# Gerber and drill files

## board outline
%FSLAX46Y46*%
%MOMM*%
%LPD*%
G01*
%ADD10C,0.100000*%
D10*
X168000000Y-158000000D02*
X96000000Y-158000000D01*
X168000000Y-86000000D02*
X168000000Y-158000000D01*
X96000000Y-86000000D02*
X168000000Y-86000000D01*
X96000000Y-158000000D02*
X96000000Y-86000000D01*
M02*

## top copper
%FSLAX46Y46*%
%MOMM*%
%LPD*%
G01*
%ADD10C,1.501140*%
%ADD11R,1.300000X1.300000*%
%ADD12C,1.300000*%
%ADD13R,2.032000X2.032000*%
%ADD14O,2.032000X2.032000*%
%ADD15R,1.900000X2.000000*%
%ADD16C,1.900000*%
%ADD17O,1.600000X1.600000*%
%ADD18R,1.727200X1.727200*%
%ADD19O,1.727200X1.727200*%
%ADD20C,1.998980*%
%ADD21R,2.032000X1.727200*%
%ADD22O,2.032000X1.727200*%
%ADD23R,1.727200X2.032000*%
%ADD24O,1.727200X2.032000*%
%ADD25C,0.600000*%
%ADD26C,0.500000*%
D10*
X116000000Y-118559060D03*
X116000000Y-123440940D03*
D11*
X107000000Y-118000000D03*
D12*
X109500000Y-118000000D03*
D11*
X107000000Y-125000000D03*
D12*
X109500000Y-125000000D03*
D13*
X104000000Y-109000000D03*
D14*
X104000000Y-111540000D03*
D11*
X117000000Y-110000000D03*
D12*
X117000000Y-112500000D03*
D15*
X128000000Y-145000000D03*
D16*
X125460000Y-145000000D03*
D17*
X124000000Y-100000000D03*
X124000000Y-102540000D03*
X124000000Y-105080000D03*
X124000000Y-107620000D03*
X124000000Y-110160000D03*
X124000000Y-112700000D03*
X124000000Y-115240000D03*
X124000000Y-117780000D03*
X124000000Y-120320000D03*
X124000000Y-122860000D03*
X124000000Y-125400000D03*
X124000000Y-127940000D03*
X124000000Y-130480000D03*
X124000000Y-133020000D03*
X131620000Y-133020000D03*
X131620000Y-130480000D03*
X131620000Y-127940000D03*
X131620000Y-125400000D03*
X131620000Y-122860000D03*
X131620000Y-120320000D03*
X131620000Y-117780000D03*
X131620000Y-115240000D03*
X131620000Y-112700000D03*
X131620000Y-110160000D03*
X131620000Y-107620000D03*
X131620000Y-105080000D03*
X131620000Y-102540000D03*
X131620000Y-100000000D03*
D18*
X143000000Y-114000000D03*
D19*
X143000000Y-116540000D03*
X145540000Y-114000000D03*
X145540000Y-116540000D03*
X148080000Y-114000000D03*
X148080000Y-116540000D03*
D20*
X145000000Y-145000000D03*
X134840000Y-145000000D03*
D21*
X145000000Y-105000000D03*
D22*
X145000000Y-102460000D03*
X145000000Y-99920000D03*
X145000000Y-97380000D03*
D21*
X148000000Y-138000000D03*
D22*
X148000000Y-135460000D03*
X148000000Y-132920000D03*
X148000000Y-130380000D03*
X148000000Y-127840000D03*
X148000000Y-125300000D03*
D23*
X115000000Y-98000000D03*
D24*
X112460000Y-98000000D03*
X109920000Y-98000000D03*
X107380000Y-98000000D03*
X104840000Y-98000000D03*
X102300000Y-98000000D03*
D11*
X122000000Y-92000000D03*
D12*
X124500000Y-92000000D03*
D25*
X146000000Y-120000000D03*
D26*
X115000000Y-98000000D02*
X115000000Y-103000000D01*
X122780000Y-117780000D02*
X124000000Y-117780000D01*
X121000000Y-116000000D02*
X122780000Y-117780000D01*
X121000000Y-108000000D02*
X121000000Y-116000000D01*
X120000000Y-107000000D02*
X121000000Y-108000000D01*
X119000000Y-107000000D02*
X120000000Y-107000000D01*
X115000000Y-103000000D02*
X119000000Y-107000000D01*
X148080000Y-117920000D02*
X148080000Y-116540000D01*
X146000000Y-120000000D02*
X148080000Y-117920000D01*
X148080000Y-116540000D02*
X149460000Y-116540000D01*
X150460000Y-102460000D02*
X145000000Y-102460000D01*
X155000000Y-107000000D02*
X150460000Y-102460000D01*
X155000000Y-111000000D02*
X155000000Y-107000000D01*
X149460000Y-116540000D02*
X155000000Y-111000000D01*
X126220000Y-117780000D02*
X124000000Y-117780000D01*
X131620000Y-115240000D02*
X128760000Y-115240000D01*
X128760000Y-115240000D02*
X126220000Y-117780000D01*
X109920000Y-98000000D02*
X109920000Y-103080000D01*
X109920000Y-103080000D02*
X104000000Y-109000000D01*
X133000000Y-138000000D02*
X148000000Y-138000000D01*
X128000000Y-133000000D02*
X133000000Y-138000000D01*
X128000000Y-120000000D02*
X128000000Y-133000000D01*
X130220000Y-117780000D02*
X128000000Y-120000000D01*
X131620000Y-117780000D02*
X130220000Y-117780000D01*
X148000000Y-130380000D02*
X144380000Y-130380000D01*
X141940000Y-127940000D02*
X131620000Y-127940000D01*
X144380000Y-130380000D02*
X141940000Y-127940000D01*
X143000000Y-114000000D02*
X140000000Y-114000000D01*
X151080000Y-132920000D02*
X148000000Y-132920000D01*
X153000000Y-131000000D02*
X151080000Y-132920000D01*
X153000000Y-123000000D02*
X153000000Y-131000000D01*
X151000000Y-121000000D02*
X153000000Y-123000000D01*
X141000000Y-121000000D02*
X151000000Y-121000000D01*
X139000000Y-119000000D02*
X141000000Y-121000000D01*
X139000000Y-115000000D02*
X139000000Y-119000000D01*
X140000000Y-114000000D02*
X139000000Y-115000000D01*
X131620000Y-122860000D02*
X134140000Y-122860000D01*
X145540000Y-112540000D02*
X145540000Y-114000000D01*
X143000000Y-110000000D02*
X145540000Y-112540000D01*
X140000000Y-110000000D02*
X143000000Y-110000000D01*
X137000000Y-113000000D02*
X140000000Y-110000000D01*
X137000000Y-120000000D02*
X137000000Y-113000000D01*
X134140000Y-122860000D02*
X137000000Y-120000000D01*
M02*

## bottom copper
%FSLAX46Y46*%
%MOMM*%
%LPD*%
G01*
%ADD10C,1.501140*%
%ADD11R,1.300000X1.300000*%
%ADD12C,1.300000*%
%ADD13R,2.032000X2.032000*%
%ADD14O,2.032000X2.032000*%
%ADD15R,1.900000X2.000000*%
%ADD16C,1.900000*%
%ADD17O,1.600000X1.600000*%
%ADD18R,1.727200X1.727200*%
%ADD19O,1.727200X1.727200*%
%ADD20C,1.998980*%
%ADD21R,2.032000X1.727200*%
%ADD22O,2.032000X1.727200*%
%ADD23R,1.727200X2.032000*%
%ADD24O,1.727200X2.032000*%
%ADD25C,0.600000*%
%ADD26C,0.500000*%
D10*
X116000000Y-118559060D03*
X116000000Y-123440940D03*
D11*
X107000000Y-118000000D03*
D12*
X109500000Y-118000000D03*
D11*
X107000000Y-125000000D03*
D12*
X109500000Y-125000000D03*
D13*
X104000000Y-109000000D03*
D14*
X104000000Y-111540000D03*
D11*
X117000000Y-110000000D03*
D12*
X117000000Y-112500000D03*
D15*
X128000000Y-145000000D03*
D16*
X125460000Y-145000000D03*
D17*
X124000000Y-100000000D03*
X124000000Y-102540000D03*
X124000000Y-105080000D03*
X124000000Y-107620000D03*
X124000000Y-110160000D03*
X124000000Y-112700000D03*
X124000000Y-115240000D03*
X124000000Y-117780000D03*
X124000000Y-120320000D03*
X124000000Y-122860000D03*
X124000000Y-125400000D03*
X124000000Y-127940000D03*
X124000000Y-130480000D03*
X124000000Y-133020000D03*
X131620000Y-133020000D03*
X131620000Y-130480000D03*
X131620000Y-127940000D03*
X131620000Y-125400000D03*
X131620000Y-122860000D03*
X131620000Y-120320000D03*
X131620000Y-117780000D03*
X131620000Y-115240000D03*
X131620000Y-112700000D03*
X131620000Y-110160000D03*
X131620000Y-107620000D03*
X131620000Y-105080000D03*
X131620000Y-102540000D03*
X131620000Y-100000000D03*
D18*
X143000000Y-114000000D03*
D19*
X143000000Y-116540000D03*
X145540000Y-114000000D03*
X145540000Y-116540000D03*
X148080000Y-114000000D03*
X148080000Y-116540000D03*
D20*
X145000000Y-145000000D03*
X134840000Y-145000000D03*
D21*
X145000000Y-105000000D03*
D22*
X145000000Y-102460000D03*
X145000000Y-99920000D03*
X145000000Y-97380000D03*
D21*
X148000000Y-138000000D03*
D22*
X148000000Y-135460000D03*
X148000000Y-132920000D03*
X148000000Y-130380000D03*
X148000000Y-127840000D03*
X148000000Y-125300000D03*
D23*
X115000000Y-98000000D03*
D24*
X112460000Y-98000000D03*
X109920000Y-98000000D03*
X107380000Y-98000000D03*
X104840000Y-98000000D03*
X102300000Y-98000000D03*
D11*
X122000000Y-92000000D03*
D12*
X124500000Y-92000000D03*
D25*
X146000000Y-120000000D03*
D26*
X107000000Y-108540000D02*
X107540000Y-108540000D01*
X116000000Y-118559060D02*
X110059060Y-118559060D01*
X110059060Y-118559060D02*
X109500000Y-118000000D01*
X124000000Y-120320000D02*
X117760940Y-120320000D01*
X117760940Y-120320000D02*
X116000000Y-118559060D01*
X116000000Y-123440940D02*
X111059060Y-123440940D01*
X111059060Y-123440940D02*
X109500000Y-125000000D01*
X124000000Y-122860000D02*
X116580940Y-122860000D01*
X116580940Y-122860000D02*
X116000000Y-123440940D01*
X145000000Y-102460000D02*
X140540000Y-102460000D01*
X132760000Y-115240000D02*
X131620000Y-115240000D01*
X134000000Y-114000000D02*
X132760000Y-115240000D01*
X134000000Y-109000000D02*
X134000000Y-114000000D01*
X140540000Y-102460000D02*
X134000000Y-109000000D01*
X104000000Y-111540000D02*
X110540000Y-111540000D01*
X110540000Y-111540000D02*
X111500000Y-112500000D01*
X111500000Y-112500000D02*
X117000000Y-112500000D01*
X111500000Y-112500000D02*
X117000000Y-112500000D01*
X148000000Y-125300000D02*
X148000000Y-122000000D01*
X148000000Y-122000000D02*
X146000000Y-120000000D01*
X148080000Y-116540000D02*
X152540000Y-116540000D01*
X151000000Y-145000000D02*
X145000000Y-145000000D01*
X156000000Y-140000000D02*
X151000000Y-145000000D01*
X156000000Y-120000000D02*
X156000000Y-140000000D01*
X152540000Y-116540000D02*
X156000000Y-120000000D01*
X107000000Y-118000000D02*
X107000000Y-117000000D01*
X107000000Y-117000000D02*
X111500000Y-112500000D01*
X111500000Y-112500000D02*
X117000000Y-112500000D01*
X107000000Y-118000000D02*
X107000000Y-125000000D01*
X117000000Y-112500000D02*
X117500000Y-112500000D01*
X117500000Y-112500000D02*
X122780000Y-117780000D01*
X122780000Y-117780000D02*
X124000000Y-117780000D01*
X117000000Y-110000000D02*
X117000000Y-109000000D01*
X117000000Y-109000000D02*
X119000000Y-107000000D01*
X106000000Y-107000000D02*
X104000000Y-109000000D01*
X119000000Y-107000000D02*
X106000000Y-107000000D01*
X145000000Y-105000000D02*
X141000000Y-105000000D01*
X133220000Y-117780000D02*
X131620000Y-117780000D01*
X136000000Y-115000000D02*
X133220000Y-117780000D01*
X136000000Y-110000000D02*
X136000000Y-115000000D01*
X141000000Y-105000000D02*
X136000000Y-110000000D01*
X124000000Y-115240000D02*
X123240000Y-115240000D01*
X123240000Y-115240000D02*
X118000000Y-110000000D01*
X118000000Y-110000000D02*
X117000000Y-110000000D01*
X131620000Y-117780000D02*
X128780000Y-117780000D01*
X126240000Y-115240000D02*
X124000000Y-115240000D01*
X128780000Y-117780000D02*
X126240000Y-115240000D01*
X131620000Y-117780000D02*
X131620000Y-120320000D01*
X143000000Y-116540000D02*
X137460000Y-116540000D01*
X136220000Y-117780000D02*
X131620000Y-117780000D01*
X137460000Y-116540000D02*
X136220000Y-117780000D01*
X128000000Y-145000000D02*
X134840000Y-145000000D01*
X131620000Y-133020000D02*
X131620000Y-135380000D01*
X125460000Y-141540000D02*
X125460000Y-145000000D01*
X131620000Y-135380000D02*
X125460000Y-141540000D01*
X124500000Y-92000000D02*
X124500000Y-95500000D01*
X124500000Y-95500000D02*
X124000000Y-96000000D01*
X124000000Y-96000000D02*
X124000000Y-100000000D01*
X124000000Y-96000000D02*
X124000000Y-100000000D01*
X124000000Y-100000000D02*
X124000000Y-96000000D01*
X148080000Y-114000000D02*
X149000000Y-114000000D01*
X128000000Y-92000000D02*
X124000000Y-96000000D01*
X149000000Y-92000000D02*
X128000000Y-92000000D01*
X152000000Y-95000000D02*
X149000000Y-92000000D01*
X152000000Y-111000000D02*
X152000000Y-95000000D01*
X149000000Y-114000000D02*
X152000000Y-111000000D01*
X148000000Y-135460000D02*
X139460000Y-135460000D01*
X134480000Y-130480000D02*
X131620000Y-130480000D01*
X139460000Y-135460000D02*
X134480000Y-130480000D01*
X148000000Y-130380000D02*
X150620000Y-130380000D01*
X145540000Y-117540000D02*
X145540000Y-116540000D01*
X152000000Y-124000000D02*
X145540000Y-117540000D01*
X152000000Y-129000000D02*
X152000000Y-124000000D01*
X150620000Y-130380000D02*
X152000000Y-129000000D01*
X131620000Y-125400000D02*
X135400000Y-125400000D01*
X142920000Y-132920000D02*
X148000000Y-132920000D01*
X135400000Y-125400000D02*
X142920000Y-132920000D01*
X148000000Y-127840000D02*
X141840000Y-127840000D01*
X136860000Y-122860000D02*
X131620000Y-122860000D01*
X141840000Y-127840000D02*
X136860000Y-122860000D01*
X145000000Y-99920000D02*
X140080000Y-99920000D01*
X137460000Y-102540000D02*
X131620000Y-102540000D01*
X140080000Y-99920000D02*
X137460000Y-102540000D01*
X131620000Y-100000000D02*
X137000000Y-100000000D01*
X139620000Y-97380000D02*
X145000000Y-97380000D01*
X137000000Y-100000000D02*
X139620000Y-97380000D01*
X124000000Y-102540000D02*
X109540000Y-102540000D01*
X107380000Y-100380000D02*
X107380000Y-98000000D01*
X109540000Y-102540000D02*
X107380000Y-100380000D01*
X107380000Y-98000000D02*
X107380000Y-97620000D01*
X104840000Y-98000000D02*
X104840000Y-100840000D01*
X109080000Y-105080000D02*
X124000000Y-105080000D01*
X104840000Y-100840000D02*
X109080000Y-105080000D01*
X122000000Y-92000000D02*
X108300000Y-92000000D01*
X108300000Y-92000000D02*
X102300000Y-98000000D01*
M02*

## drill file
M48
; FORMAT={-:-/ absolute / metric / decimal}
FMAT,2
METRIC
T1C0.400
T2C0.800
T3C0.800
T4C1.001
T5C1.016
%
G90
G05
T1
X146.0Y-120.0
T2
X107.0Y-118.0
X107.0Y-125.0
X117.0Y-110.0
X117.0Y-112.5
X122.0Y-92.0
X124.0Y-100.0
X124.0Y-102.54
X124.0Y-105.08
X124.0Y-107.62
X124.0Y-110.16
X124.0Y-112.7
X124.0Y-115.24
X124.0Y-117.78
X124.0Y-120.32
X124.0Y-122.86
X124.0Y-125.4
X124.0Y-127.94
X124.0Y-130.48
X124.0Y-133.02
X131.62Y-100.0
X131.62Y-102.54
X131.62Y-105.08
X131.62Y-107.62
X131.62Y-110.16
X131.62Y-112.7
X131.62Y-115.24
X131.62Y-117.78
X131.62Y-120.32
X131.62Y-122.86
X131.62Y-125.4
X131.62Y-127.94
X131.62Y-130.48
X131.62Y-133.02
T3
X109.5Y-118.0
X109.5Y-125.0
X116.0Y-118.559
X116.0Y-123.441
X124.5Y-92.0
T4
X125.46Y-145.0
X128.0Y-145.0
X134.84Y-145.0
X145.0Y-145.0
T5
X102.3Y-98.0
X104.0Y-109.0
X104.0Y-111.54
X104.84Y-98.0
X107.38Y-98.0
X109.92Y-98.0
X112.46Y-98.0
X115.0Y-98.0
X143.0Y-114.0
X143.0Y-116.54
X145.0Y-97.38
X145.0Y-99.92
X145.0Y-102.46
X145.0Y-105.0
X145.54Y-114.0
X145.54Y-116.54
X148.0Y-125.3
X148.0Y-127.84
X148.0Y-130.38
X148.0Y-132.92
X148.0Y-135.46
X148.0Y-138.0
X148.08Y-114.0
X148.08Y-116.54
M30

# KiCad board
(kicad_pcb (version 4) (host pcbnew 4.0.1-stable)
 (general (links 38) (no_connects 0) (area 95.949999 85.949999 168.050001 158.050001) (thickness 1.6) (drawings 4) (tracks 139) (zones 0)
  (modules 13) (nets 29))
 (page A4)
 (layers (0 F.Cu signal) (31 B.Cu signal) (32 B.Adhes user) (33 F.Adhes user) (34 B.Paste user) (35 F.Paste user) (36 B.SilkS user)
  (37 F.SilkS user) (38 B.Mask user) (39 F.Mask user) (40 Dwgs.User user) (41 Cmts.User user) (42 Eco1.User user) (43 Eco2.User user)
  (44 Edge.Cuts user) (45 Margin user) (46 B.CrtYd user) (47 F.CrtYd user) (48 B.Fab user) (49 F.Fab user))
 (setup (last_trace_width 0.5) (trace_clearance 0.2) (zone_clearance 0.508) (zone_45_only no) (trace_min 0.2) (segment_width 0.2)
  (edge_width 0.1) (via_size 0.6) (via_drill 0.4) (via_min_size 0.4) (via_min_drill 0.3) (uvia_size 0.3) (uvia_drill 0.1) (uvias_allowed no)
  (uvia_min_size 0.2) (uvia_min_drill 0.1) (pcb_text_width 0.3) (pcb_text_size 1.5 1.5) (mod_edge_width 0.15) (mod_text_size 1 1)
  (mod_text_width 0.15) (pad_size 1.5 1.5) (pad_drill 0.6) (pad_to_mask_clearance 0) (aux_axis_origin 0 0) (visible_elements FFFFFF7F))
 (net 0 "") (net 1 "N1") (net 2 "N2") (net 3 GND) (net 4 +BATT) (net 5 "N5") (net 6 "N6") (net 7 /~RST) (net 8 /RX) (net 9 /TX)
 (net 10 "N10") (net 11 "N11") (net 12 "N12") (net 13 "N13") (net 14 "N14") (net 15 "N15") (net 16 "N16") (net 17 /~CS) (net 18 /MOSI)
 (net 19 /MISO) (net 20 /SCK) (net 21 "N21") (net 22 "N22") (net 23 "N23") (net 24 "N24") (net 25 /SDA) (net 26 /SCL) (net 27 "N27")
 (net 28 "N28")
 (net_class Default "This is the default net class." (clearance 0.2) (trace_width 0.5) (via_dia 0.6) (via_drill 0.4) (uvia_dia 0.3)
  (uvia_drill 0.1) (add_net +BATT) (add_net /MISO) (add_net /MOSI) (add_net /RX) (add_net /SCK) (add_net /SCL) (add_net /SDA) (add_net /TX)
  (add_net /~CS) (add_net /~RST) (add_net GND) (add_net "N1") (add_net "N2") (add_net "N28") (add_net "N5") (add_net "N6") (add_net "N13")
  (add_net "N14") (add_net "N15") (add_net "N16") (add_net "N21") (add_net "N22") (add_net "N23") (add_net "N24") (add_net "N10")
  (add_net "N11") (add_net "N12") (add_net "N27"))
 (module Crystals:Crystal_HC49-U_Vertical (layer F.Cu) (at 116 121 270)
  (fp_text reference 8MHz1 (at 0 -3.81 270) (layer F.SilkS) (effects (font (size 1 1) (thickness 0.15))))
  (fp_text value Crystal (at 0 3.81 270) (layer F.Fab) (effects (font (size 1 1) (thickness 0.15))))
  (pad 1 thru_hole circle (at -2.44094 0 270) (size 1.50114 1.50114) (drill 0.8001) (layers *.Cu *.Mask F.SilkS) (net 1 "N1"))
  (pad 2 thru_hole circle (at 2.44094 0 270) (size 1.50114 1.50114) (drill 0.8001) (layers *.Cu *.Mask F.SilkS) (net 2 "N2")))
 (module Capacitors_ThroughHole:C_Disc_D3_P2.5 (layer F.Cu) (at 107 118)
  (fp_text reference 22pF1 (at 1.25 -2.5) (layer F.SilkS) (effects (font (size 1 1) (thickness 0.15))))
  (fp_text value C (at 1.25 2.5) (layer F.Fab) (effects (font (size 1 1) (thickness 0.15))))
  (pad 1 thru_hole rect (at 0 0) (size 1.3 1.3) (drill 0.8) (layers *.Cu *.Mask F.SilkS) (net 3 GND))
  (pad 2 thru_hole circle (at 2.5 0) (size 1.3 1.3) (drill 0.8001) (layers *.Cu *.Mask F.SilkS) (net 1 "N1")))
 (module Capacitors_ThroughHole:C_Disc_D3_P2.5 (layer F.Cu) (at 107 125)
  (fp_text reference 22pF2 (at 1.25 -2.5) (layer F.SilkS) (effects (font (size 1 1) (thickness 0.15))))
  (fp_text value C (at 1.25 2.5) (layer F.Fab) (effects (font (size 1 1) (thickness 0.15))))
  (pad 1 thru_hole rect (at 0 0) (size 1.3 1.3) (drill 0.8) (layers *.Cu *.Mask F.SilkS) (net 3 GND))
  (pad 2 thru_hole circle (at 2.5 0) (size 1.3 1.3) (drill 0.8001) (layers *.Cu *.Mask F.SilkS) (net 2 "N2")))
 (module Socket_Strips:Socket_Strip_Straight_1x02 (layer F.Cu) (at 104 109 270)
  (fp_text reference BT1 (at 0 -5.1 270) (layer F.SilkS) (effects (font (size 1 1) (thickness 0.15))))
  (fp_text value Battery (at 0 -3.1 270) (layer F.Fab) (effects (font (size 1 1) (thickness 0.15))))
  (pad 1 thru_hole rect (at 0 0 270) (size 2.032 2.032) (drill 1.016) (layers *.Cu *.Mask F.SilkS) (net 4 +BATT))
  (pad 2 thru_hole oval (at 2.54 0 270) (size 2.032 2.032) (drill 1.016) (layers *.Cu *.Mask F.SilkS) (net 3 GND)))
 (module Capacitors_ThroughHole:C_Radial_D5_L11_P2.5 (layer F.Cu) (at 117 110 270)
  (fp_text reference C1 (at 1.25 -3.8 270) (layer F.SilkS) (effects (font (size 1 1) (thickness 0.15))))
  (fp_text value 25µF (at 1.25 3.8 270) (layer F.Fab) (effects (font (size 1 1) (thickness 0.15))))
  (pad 1 thru_hole rect (at 0 0 270) (size 1.3 1.3) (drill 0.8) (layers *.Cu *.Mask F.SilkS) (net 4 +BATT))
  (pad 2 thru_hole circle (at 2.5 0 270) (size 1.3 1.3) (drill 0.8) (layers *.Cu *.Mask F.SilkS) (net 3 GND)))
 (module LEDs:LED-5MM (layer F.Cu) (at 128 145 180)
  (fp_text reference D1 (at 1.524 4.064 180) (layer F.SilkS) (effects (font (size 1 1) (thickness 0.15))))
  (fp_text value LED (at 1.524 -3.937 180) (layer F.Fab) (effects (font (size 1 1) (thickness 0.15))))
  (pad 1 thru_hole rect (at 0 0 270) (size 2 1.9) (drill 1.00076) (layers *.Cu *.Mask F.SilkS) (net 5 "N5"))
  (pad 2 thru_hole circle (at 2.54 0 180) (size 1.9 1.9) (drill 1.00076) (layers *.Cu *.Mask F.SilkS) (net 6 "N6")))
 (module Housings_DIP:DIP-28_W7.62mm (layer F.Cu) (at 124 100)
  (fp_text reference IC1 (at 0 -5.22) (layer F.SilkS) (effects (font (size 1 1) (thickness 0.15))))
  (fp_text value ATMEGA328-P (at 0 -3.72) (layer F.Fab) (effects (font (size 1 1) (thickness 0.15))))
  (pad 1 thru_hole oval (at 0 0) (size 1.6 1.6) (drill 0.8) (layers *.Cu *.Mask F.SilkS) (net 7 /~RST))
  (pad 2 thru_hole oval (at 0 2.54) (size 1.6 1.6) (drill 0.8) (layers *.Cu *.Mask F.SilkS) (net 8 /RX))
  (pad 3 thru_hole oval (at 0 5.08) (size 1.6 1.6) (drill 0.8) (layers *.Cu *.Mask F.SilkS) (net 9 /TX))
  (pad 4 thru_hole oval (at 0 7.62) (size 1.6 1.6) (drill 0.8) (layers *.Cu *.Mask F.SilkS) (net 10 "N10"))
  (pad 5 thru_hole oval (at 0 10.16) (size 1.6 1.6) (drill 0.8) (layers *.Cu *.Mask F.SilkS) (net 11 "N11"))
  (pad 6 thru_hole oval (at 0 12.7) (size 1.6 1.6) (drill 0.8) (layers *.Cu *.Mask F.SilkS) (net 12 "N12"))
  (pad 7 thru_hole oval (at 0 15.24) (size 1.6 1.6) (drill 0.8) (layers *.Cu *.Mask F.SilkS) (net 4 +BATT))
  (pad 8 thru_hole oval (at 0 17.78) (size 1.6 1.6) (drill 0.8) (layers *.Cu *.Mask F.SilkS) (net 3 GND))
  (pad 9 thru_hole oval (at 0 20.32) (size 1.6 1.6) (drill 0.8) (layers *.Cu *.Mask F.SilkS) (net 1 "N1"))
  (pad 10 thru_hole oval (at 0 22.86) (size 1.6 1.6) (drill 0.8) (layers *.Cu *.Mask F.SilkS) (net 2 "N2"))
  (pad 11 thru_hole oval (at 0 25.4) (size 1.6 1.6) (drill 0.8) (layers *.Cu *.Mask F.SilkS) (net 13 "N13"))
  (pad 12 thru_hole oval (at 0 27.94) (size 1.6 1.6) (drill 0.8) (layers *.Cu *.Mask F.SilkS) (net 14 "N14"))
  (pad 13 thru_hole oval (at 0 30.48) (size 1.6 1.6) (drill 0.8) (layers *.Cu *.Mask F.SilkS) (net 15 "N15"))
  (pad 14 thru_hole oval (at 0 33.02) (size 1.6 1.6) (drill 0.8) (layers *.Cu *.Mask F.SilkS) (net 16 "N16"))
  (pad 15 thru_hole oval (at 7.62 33.02) (size 1.6 1.6) (drill 0.8) (layers *.Cu *.Mask F.SilkS) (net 6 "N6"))
  (pad 16 thru_hole oval (at 7.62 30.48) (size 1.6 1.6) (drill 0.8) (layers *.Cu *.Mask F.SilkS) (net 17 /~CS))
  (pad 17 thru_hole oval (at 7.62 27.94) (size 1.6 1.6) (drill 0.8) (layers *.Cu *.Mask F.SilkS) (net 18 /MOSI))
  (pad 18 thru_hole oval (at 7.62 25.4) (size 1.6 1.6) (drill 0.8) (layers *.Cu *.Mask F.SilkS) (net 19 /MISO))
  (pad 19 thru_hole oval (at 7.62 22.86) (size 1.6 1.6) (drill 0.8) (layers *.Cu *.Mask F.SilkS) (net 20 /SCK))
  (pad 20 thru_hole oval (at 7.62 20.32) (size 1.6 1.6) (drill 0.8) (layers *.Cu *.Mask F.SilkS) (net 4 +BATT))
  (pad 21 thru_hole oval (at 7.62 17.78) (size 1.6 1.6) (drill 0.8) (layers *.Cu *.Mask F.SilkS) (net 4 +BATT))
  (pad 22 thru_hole oval (at 7.62 15.24) (size 1.6 1.6) (drill 0.8) (layers *.Cu *.Mask F.SilkS) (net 3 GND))
  (pad 23 thru_hole oval (at 7.62 12.7) (size 1.6 1.6) (drill 0.8) (layers *.Cu *.Mask F.SilkS) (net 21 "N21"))
  (pad 24 thru_hole oval (at 7.62 10.16) (size 1.6 1.6) (drill 0.8) (layers *.Cu *.Mask F.SilkS) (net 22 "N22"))
  (pad 25 thru_hole oval (at 7.62 7.62) (size 1.6 1.6) (drill 0.8) (layers *.Cu *.Mask F.SilkS) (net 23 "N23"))
  (pad 26 thru_hole oval (at 7.62 5.08) (size 1.6 1.6) (drill 0.8) (layers *.Cu *.Mask F.SilkS) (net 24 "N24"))
  (pad 27 thru_hole oval (at 7.62 2.54) (size 1.6 1.6) (drill 0.8) (layers *.Cu *.Mask F.SilkS) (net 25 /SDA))
  (pad 28 thru_hole oval (at 7.62 0) (size 1.6 1.6) (drill 0.8) (layers *.Cu *.Mask F.SilkS) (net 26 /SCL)))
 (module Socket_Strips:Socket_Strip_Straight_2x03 (layer F.Cu) (at 143 114)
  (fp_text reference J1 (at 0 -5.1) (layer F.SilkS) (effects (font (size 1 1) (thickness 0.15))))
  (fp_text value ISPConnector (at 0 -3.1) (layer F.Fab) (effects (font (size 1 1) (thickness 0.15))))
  (pad 1 thru_hole rect (at 0 0) (size 1.7272 1.7272) (drill 1.016) (layers *.Cu *.Mask F.SilkS) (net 19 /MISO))
  (pad 2 thru_hole oval (at 0 2.54) (size 1.7272 1.7272) (drill 1.016) (layers *.Cu *.Mask F.SilkS) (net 4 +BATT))
  (pad 3 thru_hole oval (at 2.54 0) (size 1.7272 1.7272) (drill 1.016) (layers *.Cu *.Mask F.SilkS) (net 20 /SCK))
  (pad 4 thru_hole oval (at 2.54 2.54) (size 1.7272 1.7272) (drill 1.016) (layers *.Cu *.Mask F.SilkS) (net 18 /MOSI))
  (pad 5 thru_hole oval (at 5.08 0) (size 1.7272 1.7272) (drill 1.016) (layers *.Cu *.Mask F.SilkS) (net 7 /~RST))
  (pad 6 thru_hole oval (at 5.08 2.54) (size 1.7272 1.7272) (drill 1.016) (layers *.Cu *.Mask F.SilkS) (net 3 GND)))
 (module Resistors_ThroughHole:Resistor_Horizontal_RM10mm (layer F.Cu) (at 145 145 180)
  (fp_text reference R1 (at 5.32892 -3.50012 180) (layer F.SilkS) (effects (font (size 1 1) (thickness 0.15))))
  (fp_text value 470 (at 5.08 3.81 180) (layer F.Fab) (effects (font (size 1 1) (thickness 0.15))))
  (pad 1 thru_hole circle (at 0 0 180) (size 1.99898 1.99898) (drill 1.00076) (layers *.Cu *.SilkS *.Mask) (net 3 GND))
  (pad 2 thru_hole circle (at 10.16 0 180) (size 1.99898 1.99898) (drill 1.00076) (layers *.Cu *.SilkS *.Mask) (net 5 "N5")))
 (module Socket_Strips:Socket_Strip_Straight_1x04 (layer F.Cu) (at 145 105 90)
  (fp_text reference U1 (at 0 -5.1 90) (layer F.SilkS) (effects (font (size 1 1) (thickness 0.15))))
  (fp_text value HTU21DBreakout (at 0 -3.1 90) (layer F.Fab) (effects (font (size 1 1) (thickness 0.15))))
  (pad 1 thru_hole rect (at 0 0 90) (size 1.7272 2.032) (drill 1.016) (layers *.Cu *.Mask F.SilkS) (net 4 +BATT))
  (pad 2 thru_hole oval (at 2.54 0 90) (size 1.7272 2.032) (drill 1.016) (layers *.Cu *.Mask F.SilkS) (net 3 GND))
  (pad 3 thru_hole oval (at 5.08 0 90) (size 1.7272 2.032) (drill 1.016) (layers *.Cu *.Mask F.SilkS) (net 25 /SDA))
  (pad 4 thru_hole oval (at 7.62 0 90) (size 1.7272 2.032) (drill 1.016) (layers *.Cu *.Mask F.SilkS) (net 26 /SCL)))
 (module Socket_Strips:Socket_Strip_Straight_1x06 (layer F.Cu) (at 148 138 90)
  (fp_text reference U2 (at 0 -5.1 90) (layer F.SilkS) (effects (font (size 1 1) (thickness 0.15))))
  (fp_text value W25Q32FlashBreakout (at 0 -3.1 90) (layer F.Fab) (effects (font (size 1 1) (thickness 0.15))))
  (pad 1 thru_hole rect (at 0 0 90) (size 1.7272 2.032) (drill 1.016) (layers *.Cu *.Mask F.SilkS) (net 4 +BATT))
  (pad 2 thru_hole oval (at 2.54 0 90) (size 1.7272 2.032) (drill 1.016) (layers *.Cu *.Mask F.SilkS) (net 17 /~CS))
  (pad 3 thru_hole oval (at 5.08 0 90) (size 1.7272 2.032) (drill 1.016) (layers *.Cu *.Mask F.SilkS) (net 19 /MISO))
  (pad 4 thru_hole oval (at 7.62 0 90) (size 1.7272 2.032) (drill 1.016) (layers *.Cu *.Mask F.SilkS) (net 18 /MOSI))
  (pad 5 thru_hole oval (at 10.16 0 90) (size 1.7272 2.032) (drill 1.016) (layers *.Cu *.Mask F.SilkS) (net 20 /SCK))
  (pad 6 thru_hole oval (at 12.7 0 90) (size 1.7272 2.032) (drill 1.016) (layers *.Cu *.Mask F.SilkS) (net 3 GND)))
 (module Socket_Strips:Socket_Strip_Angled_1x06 (layer F.Cu) (at 115 98 180)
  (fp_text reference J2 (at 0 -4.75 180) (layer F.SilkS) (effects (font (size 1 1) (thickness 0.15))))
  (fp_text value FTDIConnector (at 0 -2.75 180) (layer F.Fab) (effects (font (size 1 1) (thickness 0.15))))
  (pad 1 thru_hole rect (at 0 0 180) (size 1.7272 2.032) (drill 1.016) (layers *.Cu *.Mask F.SilkS) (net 3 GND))
  (pad 2 thru_hole oval (at 2.54 0 180) (size 1.7272 2.032) (drill 1.016) (layers *.Cu *.Mask F.SilkS) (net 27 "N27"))
  (pad 3 thru_hole oval (at 5.08 0 180) (size 1.7272 2.032) (drill 1.016) (layers *.Cu *.Mask F.SilkS) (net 4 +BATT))
  (pad 4 thru_hole oval (at 7.62 0 180) (size 1.7272 2.032) (drill 1.016) (layers *.Cu *.Mask F.SilkS) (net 8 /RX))
  (pad 5 thru_hole oval (at 10.16 0 180) (size 1.7272 2.032) (drill 1.016) (layers *.Cu *.Mask F.SilkS) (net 9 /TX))
  (pad 6 thru_hole oval (at 12.7 0 180) (size 1.7272 2.032) (drill 1.016) (layers *.Cu *.Mask F.SilkS) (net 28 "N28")))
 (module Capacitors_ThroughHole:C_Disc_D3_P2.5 (layer F.Cu) (at 122 92)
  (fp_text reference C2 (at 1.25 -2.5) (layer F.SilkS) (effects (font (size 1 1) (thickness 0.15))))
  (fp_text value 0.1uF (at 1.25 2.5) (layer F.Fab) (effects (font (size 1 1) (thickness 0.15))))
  (pad 1 thru_hole rect (at 0 0) (size 1.3 1.3) (drill 0.8) (layers *.Cu *.Mask F.SilkS) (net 28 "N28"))
  (pad 2 thru_hole circle (at 2.5 0) (size 1.3 1.3) (drill 0.8001) (layers *.Cu *.Mask F.SilkS) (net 7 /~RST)))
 (gr_line (start 168 158) (end 96 158) (angle 90) (layer Edge.Cuts) (width 0.1))
 (gr_line (start 168 86) (end 168 158) (angle 90) (layer Edge.Cuts) (width 0.1))
 (gr_line (start 96 86) (end 168 86) (angle 90) (layer Edge.Cuts) (width 0.1))
 (gr_line (start 96 158) (end 96 86) (angle 90) (layer Edge.Cuts) (width 0.1))
 (segment (start 107 108.54) (end 107.54 108.54) (width 0.5) (layer B.Cu) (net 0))
 (segment (start 116 118.55906) (end 110.05906 118.55906) (width 0.5) (layer B.Cu) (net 1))
 (segment (start 110.05906 118.55906) (end 109.5 118) (width 0.5) (layer B.Cu) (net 1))
 (segment (start 124 120.32) (end 117.76094 120.32) (width 0.5) (layer B.Cu) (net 1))
 (segment (start 117.76094 120.32) (end 116 118.55906) (width 0.5) (layer B.Cu) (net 1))
 (segment (start 116 123.44094) (end 111.05906 123.44094) (width 0.5) (layer B.Cu) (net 2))
 (segment (start 111.05906 123.44094) (end 109.5 125) (width 0.5) (layer B.Cu) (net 2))
 (segment (start 124 122.86) (end 116.58094 122.86) (width 0.5) (layer B.Cu) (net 2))
 (segment (start 116.58094 122.86) (end 116 123.44094) (width 0.5) (layer B.Cu) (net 2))
 (segment (start 145 102.46) (end 140.54 102.46) (width 0.5) (layer B.Cu) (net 3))
 (segment (start 132.76 115.24) (end 131.62 115.24) (width 0.5) (layer B.Cu) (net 3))
 (segment (start 134 114) (end 132.76 115.24) (width 0.5) (layer B.Cu) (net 3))
 (segment (start 134 109) (end 134 114) (width 0.5) (layer B.Cu) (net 3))
 (segment (start 140.54 102.46) (end 134 109) (width 0.5) (layer B.Cu) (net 3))
 (segment (start 115 98) (end 115 103) (width 0.5) (layer F.Cu) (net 3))
 (segment (start 122.78 117.78) (end 124 117.78) (width 0.5) (layer F.Cu) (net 3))
 (segment (start 121 116) (end 122.78 117.78) (width 0.5) (layer F.Cu) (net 3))
 (segment (start 121 108) (end 121 116) (width 0.5) (layer F.Cu) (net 3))
 (segment (start 120 107) (end 121 108) (width 0.5) (layer F.Cu) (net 3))
 (segment (start 119 107) (end 120 107) (width 0.5) (layer F.Cu) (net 3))
 (segment (start 115 103) (end 119 107) (width 0.5) (layer F.Cu) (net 3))
 (segment (start 104 111.54) (end 110.54 111.54) (width 0.5) (layer B.Cu) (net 3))
 (segment (start 110.54 111.54) (end 111.5 112.5) (width 0.5) (layer B.Cu) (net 3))
 (segment (start 111.5 112.5) (end 117 112.5) (width 0.5) (layer B.Cu) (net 3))
 (segment (start 111.5 112.5) (end 117 112.5) (width 0.5) (layer B.Cu) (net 3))
 (segment (start 148 125.3) (end 148 122) (width 0.5) (layer B.Cu) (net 3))
 (segment (start 148.08 117.92) (end 148.08 116.54) (width 0.5) (layer F.Cu) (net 3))
 (segment (start 146 120) (end 148.08 117.92) (width 0.5) (layer F.Cu) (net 3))
 (via (at 146 120) (size 0.6) (drill 0.4) (layers F.Cu B.Cu) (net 3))
 (segment (start 148 122) (end 146 120) (width 0.5) (layer B.Cu) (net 3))
 (segment (start 148.08 116.54) (end 152.54 116.54) (width 0.5) (layer B.Cu) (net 3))
 (segment (start 151 145) (end 145 145) (width 0.5) (layer B.Cu) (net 3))
 (segment (start 156 140) (end 151 145) (width 0.5) (layer B.Cu) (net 3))
 (segment (start 156 120) (end 156 140) (width 0.5) (layer B.Cu) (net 3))
 (segment (start 152.54 116.54) (end 156 120) (width 0.5) (layer B.Cu) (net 3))
 (segment (start 148.08 116.54) (end 149.46 116.54) (width 0.5) (layer F.Cu) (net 3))
 (segment (start 150.46 102.46) (end 145 102.46) (width 0.5) (layer F.Cu) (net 3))
 (segment (start 155 107) (end 150.46 102.46) (width 0.5) (layer F.Cu) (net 3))
 (segment (start 155 111) (end 155 107) (width 0.5) (layer F.Cu) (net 3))
 (segment (start 149.46 116.54) (end 155 111) (width 0.5) (layer F.Cu) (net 3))
 (segment (start 107 118) (end 107 117) (width 0.5) (layer B.Cu) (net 3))
 (segment (start 107 117) (end 111.5 112.5) (width 0.5) (layer B.Cu) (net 3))
 (segment (start 111.5 112.5) (end 117 112.5) (width 0.5) (layer B.Cu) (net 3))
 (segment (start 107 118) (end 107 125) (width 0.5) (layer B.Cu) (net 3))
 (segment (start 117 112.5) (end 117.5 112.5) (width 0.5) (layer B.Cu) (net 3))
 (segment (start 117.5 112.5) (end 122.78 117.78) (width 0.5) (layer B.Cu) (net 3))
 (segment (start 122.78 117.78) (end 124 117.78) (width 0.5) (layer B.Cu) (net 3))
 (segment (start 126.22 117.78) (end 124 117.78) (width 0.5) (layer F.Cu) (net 3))
 (segment (start 131.62 115.24) (end 128.76 115.24) (width 0.5) (layer F.Cu) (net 3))
 (segment (start 128.76 115.24) (end 126.22 117.78) (width 0.5) (layer F.Cu) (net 3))
 (segment (start 109.92 98) (end 109.92 103.08) (width 0.5) (layer F.Cu) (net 4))
 (segment (start 109.92 103.08) (end 104 109) (width 0.5) (layer F.Cu) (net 4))
 (segment (start 117 110) (end 117 109) (width 0.5) (layer B.Cu) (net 4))
 (segment (start 117 109) (end 119 107) (width 0.5) (layer B.Cu) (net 4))
 (segment (start 106 107) (end 104 109) (width 0.5) (layer B.Cu) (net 4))
 (segment (start 119 107) (end 106 107) (width 0.5) (layer B.Cu) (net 4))
 (segment (start 133 138) (end 148 138) (width 0.5) (layer F.Cu) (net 4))
 (segment (start 128 133) (end 133 138) (width 0.5) (layer F.Cu) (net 4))
 (segment (start 128 120) (end 128 133) (width 0.5) (layer F.Cu) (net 4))
 (segment (start 130.22 117.78) (end 128 120) (width 0.5) (layer F.Cu) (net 4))
 (segment (start 131.62 117.78) (end 130.22 117.78) (width 0.5) (layer F.Cu) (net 4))
 (segment (start 145 105) (end 141 105) (width 0.5) (layer B.Cu) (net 4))
 (segment (start 133.22 117.78) (end 131.62 117.78) (width 0.5) (layer B.Cu) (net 4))
 (segment (start 136 115) (end 133.22 117.78) (width 0.5) (layer B.Cu) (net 4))
 (segment (start 136 110) (end 136 115) (width 0.5) (layer B.Cu) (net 4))
 (segment (start 141 105) (end 136 110) (width 0.5) (layer B.Cu) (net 4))
 (segment (start 124 115.24) (end 123.24 115.24) (width 0.5) (layer B.Cu) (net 4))
 (segment (start 123.24 115.24) (end 118 110) (width 0.5) (layer B.Cu) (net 4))
 (segment (start 118 110) (end 117 110) (width 0.5) (layer B.Cu) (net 4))
 (segment (start 131.62 117.78) (end 128.78 117.78) (width 0.5) (layer B.Cu) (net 4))
 (segment (start 126.24 115.24) (end 124 115.24) (width 0.5) (layer B.Cu) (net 4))
 (segment (start 128.78 117.78) (end 126.24 115.24) (width 0.5) (layer B.Cu) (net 4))
 (segment (start 131.62 117.78) (end 131.62 120.32) (width 0.5) (layer B.Cu) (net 4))
 (segment (start 143 116.54) (end 137.46 116.54) (width 0.5) (layer B.Cu) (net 4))
 (segment (start 136.22 117.78) (end 131.62 117.78) (width 0.5) (layer B.Cu) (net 4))
 (segment (start 137.46 116.54) (end 136.22 117.78) (width 0.5) (layer B.Cu) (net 4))
 (segment (start 128 145) (end 134.84 145) (width 0.5) (layer B.Cu) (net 5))
 (segment (start 131.62 133.02) (end 131.62 135.38) (width 0.5) (layer B.Cu) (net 6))
 (segment (start 125.46 141.54) (end 125.46 145) (width 0.5) (layer B.Cu) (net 6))
 (segment (start 131.62 135.38) (end 125.46 141.54) (width 0.5) (layer B.Cu) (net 6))
 (segment (start 124.5 92) (end 124.5 95.5) (width 0.5) (layer B.Cu) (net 7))
 (segment (start 124.5 95.5) (end 124 96) (width 0.5) (layer B.Cu) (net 7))
 (segment (start 124 96) (end 124 100) (width 0.5) (layer B.Cu) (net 7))
 (segment (start 124 96) (end 124 100) (width 0.5) (layer B.Cu) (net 7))
 (segment (start 124 100) (end 124 96) (width 0.5) (layer B.Cu) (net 7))
 (segment (start 148.08 114) (end 149 114) (width 0.5) (layer B.Cu) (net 7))
 (segment (start 128 92) (end 124 96) (width 0.5) (layer B.Cu) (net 7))
 (segment (start 149 92) (end 128 92) (width 0.5) (layer B.Cu) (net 7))
 (segment (start 152 95) (end 149 92) (width 0.5) (layer B.Cu) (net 7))
 (segment (start 152 111) (end 152 95) (width 0.5) (layer B.Cu) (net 7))
 (segment (start 149 114) (end 152 111) (width 0.5) (layer B.Cu) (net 7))
 (segment (start 148 135.46) (end 139.46 135.46) (width 0.5) (layer B.Cu) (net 17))
 (segment (start 134.48 130.48) (end 131.62 130.48) (width 0.5) (layer B.Cu) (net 17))
 (segment (start 139.46 135.46) (end 134.48 130.48) (width 0.5) (layer B.Cu) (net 17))
 (segment (start 148 130.38) (end 150.62 130.38) (width 0.5) (layer B.Cu) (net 18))
 (segment (start 145.54 117.54) (end 145.54 116.54) (width 0.5) (layer B.Cu) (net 18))
 (segment (start 152 124) (end 145.54 117.54) (width 0.5) (layer B.Cu) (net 18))
 (segment (start 152 129) (end 152 124) (width 0.5) (layer B.Cu) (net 18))
 (segment (start 150.62 130.38) (end 152 129) (width 0.5) (layer B.Cu) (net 18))
 (segment (start 148 130.38) (end 144.38 130.38) (width 0.5) (layer F.Cu) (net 18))
 (segment (start 141.94 127.94) (end 131.62 127.94) (width 0.5) (layer F.Cu) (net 18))
 (segment (start 144.38 130.38) (end 141.94 127.94) (width 0.5) (layer F.Cu) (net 18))
 (segment (start 143 114) (end 140 114) (width 0.5) (layer F.Cu) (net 19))
 (segment (start 151.08 132.92) (end 148 132.92) (width 0.5) (layer F.Cu) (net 19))
 (segment (start 153 131) (end 151.08 132.92) (width 0.5) (layer F.Cu) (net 19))
 (segment (start 153 123) (end 153 131) (width 0.5) (layer F.Cu) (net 19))
 (segment (start 151 121) (end 153 123) (width 0.5) (layer F.Cu) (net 19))
 (segment (start 141 121) (end 151 121) (width 0.5) (layer F.Cu) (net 19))
 (segment (start 139 119) (end 141 121) (width 0.5) (layer F.Cu) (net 19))
 (segment (start 139 115) (end 139 119) (width 0.5) (layer F.Cu) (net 19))
 (segment (start 140 114) (end 139 115) (width 0.5) (layer F.Cu) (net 19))
 (segment (start 131.62 125.4) (end 135.4 125.4) (width 0.5) (layer B.Cu) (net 19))
 (segment (start 142.92 132.92) (end 148 132.92) (width 0.5) (layer B.Cu) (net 19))
 (segment (start 135.4 125.4) (end 142.92 132.92) (width 0.5) (layer B.Cu) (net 19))
 (segment (start 131.62 122.86) (end 134.14 122.86) (width 0.5) (layer F.Cu) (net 20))
 (segment (start 145.54 112.54) (end 145.54 114) (width 0.5) (layer F.Cu) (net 20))
 (segment (start 143 110) (end 145.54 112.54) (width 0.5) (layer F.Cu) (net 20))
 (segment (start 140 110) (end 143 110) (width 0.5) (layer F.Cu) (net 20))
 (segment (start 137 113) (end 140 110) (width 0.5) (layer F.Cu) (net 20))
 (segment (start 137 120) (end 137 113) (width 0.5) (layer F.Cu) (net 20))
 (segment (start 134.14 122.86) (end 137 120) (width 0.5) (layer F.Cu) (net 20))
 (segment (start 148 127.84) (end 141.84 127.84) (width 0.5) (layer B.Cu) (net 20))
 (segment (start 136.86 122.86) (end 131.62 122.86) (width 0.5) (layer B.Cu) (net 20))
 (segment (start 141.84 127.84) (end 136.86 122.86) (width 0.5) (layer B.Cu) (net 20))
 (segment (start 145 99.92) (end 140.08 99.92) (width 0.5) (layer B.Cu) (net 25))
 (segment (start 137.46 102.54) (end 131.62 102.54) (width 0.5) (layer B.Cu) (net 25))
 (segment (start 140.08 99.92) (end 137.46 102.54) (width 0.5) (layer B.Cu) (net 25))
 (segment (start 131.62 100) (end 137 100) (width 0.5) (layer B.Cu) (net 26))
 (segment (start 139.62 97.38) (end 145 97.38) (width 0.5) (layer B.Cu) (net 26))
 (segment (start 137 100) (end 139.62 97.38) (width 0.5) (layer B.Cu) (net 26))
 (segment (start 124 102.54) (end 109.54 102.54) (width 0.5) (layer B.Cu) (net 8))
 (segment (start 107.38 100.38) (end 107.38 98) (width 0.5) (layer B.Cu) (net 8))
 (segment (start 109.54 102.54) (end 107.38 100.38) (width 0.5) (layer B.Cu) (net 8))
 (segment (start 107.38 98) (end 107.38 97.62) (width 0.5) (layer B.Cu) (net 8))
 (segment (start 104.84 98) (end 104.84 100.84) (width 0.5) (layer B.Cu) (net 9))
 (segment (start 109.08 105.08) (end 124 105.08) (width 0.5) (layer B.Cu) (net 9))
 (segment (start 104.84 100.84) (end 109.08 105.08) (width 0.5) (layer B.Cu) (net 9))
 (segment (start 122 92) (end 108.3 92) (width 0.5) (layer B.Cu) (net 28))
 (segment (start 108.3 92) (end 102.3 98) (width 0.5) (layer B.Cu) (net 28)))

